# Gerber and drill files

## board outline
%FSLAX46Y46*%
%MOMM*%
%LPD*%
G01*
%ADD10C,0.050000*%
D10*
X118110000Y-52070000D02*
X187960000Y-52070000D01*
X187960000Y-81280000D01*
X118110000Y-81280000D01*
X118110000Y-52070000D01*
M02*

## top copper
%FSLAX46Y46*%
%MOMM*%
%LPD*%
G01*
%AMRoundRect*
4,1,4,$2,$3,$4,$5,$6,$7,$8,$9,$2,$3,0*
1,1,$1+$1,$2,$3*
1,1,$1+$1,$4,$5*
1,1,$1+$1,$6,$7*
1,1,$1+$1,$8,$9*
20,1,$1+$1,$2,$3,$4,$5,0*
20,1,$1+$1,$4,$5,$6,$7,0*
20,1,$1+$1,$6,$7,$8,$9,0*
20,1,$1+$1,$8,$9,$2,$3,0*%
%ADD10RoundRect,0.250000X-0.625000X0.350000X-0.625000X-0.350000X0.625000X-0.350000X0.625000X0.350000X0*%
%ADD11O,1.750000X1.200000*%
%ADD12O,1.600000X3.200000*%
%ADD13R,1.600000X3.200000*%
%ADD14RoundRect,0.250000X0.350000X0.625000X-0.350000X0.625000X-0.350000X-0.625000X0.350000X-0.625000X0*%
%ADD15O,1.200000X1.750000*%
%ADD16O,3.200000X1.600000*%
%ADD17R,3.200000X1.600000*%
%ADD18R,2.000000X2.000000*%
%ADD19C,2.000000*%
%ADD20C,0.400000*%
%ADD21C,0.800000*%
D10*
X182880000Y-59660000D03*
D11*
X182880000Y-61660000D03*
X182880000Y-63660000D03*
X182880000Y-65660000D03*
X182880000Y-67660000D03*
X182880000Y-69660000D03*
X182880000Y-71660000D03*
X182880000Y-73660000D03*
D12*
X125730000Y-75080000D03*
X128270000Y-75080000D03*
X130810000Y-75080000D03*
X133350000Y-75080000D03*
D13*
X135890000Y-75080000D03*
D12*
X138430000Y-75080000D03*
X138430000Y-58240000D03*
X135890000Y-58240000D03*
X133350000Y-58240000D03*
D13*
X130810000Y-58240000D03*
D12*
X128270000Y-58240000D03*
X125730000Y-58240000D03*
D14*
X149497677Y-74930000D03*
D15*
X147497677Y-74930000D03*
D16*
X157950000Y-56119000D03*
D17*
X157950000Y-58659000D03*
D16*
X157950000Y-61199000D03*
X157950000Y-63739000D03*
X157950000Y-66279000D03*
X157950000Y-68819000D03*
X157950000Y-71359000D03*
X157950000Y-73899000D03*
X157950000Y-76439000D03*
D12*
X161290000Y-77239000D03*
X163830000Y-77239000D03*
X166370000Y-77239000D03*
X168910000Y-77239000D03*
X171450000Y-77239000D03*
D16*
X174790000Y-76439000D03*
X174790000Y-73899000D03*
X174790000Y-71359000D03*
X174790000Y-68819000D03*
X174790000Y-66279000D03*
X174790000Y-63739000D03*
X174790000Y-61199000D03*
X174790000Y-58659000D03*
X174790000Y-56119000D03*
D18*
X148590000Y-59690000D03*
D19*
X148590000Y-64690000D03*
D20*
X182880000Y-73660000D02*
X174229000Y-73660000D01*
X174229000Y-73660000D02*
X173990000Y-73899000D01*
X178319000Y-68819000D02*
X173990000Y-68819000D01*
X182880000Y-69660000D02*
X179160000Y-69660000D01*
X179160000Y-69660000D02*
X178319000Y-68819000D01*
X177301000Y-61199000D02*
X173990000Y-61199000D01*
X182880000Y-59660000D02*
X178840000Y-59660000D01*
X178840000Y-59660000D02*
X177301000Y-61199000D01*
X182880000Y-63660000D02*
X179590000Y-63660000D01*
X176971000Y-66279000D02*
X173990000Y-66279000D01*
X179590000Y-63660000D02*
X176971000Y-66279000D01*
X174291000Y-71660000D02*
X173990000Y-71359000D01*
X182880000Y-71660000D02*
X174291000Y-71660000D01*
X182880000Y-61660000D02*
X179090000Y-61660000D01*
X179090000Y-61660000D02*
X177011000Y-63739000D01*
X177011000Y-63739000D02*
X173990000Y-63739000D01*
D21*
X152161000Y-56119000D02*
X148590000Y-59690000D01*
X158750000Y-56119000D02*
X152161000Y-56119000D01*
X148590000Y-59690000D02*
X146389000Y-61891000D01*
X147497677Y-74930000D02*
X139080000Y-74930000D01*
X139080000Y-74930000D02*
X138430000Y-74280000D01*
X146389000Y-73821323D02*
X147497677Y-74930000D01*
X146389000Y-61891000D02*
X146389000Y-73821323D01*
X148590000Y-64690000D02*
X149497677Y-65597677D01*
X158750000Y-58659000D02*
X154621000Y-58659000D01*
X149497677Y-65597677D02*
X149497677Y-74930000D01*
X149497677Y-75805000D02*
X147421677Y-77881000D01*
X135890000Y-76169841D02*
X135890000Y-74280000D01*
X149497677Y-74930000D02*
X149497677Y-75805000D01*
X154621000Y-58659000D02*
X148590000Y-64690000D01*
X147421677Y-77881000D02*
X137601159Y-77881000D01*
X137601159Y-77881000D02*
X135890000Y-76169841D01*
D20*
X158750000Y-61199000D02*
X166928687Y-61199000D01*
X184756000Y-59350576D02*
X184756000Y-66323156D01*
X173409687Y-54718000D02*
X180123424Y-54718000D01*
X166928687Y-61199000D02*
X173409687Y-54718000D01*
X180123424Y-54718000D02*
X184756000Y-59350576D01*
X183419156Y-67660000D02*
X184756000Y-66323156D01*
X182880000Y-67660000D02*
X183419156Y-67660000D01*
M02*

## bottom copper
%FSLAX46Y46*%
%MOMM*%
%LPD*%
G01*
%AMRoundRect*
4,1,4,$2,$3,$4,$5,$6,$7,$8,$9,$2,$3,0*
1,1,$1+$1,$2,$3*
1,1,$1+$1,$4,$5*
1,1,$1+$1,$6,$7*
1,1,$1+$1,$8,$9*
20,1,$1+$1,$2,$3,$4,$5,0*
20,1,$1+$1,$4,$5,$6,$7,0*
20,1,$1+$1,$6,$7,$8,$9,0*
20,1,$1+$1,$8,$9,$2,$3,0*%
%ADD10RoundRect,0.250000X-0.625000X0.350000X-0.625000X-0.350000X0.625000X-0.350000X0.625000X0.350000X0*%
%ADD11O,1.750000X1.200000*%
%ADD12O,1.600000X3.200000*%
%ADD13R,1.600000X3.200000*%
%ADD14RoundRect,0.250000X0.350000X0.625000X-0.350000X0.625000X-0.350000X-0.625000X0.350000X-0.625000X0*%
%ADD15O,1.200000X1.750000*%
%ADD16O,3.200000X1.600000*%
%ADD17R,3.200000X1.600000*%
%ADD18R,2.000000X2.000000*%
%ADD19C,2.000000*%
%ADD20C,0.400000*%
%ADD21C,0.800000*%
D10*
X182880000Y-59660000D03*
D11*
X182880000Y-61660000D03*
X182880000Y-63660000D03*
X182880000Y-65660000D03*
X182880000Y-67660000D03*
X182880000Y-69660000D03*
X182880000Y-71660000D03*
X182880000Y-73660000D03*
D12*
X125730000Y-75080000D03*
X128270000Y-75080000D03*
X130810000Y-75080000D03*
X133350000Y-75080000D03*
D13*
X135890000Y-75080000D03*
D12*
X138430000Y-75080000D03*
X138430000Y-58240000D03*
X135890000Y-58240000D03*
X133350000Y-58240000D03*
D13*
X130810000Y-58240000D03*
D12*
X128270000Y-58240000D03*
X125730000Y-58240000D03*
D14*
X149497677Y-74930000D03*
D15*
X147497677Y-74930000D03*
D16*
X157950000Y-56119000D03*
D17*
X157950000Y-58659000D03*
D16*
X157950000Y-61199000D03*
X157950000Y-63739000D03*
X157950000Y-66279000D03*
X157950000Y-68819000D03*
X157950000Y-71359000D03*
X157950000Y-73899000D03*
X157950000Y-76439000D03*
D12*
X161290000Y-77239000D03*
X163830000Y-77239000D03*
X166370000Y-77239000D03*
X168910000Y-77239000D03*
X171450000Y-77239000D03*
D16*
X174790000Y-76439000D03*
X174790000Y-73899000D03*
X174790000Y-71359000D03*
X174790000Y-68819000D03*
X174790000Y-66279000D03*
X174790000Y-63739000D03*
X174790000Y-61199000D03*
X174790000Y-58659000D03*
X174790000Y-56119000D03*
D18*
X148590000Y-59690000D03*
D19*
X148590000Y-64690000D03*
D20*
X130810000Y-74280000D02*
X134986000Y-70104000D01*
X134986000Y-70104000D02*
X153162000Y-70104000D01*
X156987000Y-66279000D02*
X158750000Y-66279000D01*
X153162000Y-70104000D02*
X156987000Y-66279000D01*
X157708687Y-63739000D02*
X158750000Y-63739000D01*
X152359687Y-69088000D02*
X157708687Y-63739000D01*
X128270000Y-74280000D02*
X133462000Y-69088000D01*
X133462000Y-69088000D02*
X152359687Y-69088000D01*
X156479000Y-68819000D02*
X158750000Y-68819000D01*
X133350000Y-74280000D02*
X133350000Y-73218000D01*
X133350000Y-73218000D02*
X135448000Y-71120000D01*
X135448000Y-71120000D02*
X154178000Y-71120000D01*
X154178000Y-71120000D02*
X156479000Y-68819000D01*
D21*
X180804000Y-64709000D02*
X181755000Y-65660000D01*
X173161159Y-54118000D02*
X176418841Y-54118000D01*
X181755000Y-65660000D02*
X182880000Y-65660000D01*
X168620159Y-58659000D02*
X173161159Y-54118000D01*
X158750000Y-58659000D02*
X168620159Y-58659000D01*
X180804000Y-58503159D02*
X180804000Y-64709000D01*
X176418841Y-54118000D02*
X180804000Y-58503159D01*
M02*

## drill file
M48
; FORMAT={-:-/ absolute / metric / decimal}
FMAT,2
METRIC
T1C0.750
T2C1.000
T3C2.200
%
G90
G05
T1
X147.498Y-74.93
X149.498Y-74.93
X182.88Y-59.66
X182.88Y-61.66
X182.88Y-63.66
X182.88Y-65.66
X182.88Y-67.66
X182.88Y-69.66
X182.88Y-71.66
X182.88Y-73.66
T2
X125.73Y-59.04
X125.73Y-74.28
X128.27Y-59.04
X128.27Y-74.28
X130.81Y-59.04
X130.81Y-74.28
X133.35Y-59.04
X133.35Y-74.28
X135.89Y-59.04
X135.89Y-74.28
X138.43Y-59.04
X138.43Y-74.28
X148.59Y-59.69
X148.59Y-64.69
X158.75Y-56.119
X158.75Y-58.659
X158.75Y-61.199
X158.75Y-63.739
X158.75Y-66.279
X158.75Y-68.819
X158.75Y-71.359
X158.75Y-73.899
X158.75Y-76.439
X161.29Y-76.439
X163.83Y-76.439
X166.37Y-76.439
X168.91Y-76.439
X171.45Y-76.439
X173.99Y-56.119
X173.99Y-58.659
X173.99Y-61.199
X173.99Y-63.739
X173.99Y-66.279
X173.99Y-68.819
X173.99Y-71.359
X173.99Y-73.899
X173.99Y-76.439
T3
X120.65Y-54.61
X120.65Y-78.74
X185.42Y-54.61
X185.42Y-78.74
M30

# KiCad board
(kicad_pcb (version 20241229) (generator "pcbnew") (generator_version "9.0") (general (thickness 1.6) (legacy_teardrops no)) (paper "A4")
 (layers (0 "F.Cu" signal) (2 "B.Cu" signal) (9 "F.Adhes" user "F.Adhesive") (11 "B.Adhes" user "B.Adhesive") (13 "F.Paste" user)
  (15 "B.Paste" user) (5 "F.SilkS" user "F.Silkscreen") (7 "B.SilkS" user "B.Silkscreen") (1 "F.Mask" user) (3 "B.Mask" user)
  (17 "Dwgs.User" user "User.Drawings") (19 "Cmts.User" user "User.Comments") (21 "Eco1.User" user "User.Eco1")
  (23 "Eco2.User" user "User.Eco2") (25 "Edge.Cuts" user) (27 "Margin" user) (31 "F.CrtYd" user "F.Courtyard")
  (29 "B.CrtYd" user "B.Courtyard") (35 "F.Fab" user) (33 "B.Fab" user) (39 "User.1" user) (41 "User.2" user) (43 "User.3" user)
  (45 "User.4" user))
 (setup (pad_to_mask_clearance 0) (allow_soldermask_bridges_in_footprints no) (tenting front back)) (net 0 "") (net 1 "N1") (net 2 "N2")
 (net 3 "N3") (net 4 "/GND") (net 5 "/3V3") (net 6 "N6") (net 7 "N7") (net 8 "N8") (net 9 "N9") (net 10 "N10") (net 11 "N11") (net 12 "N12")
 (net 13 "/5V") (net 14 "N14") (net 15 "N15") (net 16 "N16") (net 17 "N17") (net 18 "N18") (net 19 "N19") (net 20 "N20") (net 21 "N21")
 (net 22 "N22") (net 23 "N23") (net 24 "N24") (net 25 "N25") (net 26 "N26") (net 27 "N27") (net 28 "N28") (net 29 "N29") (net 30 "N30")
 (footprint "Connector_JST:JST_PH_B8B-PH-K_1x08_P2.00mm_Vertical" (layer "F.Cu") (at 182.88 59.66 -90)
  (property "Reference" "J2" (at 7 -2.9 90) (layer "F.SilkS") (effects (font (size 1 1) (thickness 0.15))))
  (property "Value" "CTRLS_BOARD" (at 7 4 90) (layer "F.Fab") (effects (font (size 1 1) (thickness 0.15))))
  (pad "1" thru_hole roundrect (at 0 0 270) (size 1.2 1.75) (drill 0.75) (layers "*.Cu" "*.Mask") (remove_unused_layers no)
   (roundrect_rratio 0.208333) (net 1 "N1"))
  (pad "2" thru_hole oval (at 2 0 270) (size 1.2 1.75) (drill 0.75) (layers "*.Cu" "*.Mask") (remove_unused_layers no) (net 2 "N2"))
  (pad "3" thru_hole oval (at 4 0 270) (size 1.2 1.75) (drill 0.75) (layers "*.Cu" "*.Mask") (remove_unused_layers no) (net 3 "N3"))
  (pad "4" thru_hole oval (at 6 0 270) (size 1.2 1.75) (drill 0.75) (layers "*.Cu" "*.Mask") (remove_unused_layers no) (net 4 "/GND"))
  (pad "5" thru_hole oval (at 8 0 270) (size 1.2 1.75) (drill 0.75) (layers "*.Cu" "*.Mask") (remove_unused_layers no) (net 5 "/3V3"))
  (pad "6" thru_hole oval (at 10 0 270) (size 1.2 1.75) (drill 0.75) (layers "*.Cu" "*.Mask") (remove_unused_layers no) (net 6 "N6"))
  (pad "7" thru_hole oval (at 12 0 270) (size 1.2 1.75) (drill 0.75) (layers "*.Cu" "*.Mask") (remove_unused_layers no) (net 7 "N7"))
  (pad "8" thru_hole oval (at 14 0 270) (size 1.2 1.75) (drill 0.75) (layers "*.Cu" "*.Mask") (remove_unused_layers no) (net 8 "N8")))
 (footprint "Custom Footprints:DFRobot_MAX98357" (layer "F.Cu") (at 140.97 66.66 90)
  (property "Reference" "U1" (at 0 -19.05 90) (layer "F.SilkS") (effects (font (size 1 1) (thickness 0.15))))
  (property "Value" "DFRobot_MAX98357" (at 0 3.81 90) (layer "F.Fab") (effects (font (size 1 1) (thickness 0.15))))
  (pad "1" thru_hole oval (at -7.62 -15.24 90) (size 3.2 1.6) (drill 1 (offset -0.8 0)) (layers "*.Cu" "*.Mask") (remove_unused_layers no)
   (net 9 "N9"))
  (pad "2" thru_hole oval (at -7.62 -12.7 90) (size 3.2 1.6) (drill 1 (offset -0.8 0)) (layers "*.Cu" "*.Mask") (remove_unused_layers no)
   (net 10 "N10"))
  (pad "3" thru_hole oval (at -7.62 -10.16 90) (size 3.2 1.6) (drill 1 (offset -0.8 0)) (layers "*.Cu" "*.Mask") (remove_unused_layers no)
   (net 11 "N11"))
  (pad "4" thru_hole oval (at -7.62 -7.62 90) (size 3.2 1.6) (drill 1 (offset -0.8 0)) (layers "*.Cu" "*.Mask") (remove_unused_layers no)
   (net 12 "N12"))
  (pad "5" thru_hole rect (at -7.62 -5.08 90) (size 3.2 1.6) (drill 1 (offset -0.8 0)) (layers "*.Cu" "*.Mask") (remove_unused_layers no)
   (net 4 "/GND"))
  (pad "6" thru_hole oval (at -7.62 -2.54 90) (size 3.2 1.6) (drill 1 (offset -0.8 0)) (layers "*.Cu" "*.Mask") (remove_unused_layers no)
   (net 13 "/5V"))
  (pad "7" thru_hole oval (at 7.62 -2.54 90) (size 3.2 1.6) (drill 1 (offset 0.8 0)) (layers "*.Cu" "*.Mask") (remove_unused_layers no)
   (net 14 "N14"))
  (pad "8" thru_hole oval (at 7.62 -5.08 90) (size 3.2 1.6) (drill 1 (offset 0.8 0)) (layers "*.Cu" "*.Mask") (remove_unused_layers no)
   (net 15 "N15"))
  (pad "9" thru_hole oval (at 7.62 -7.62 90) (size 3.2 1.6) (drill 1 (offset 0.8 0)) (layers "*.Cu" "*.Mask") (remove_unused_layers no)
   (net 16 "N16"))
  (pad "10" thru_hole rect (at 7.62 -10.16 90) (size 3.2 1.6) (drill 1 (offset 0.8 0)) (layers "*.Cu" "*.Mask") (remove_unused_layers no)
   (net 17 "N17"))
  (pad "11" thru_hole oval (at 7.62 -12.7 90) (size 3.2 1.6) (drill 1 (offset 0.8 0)) (layers "*.Cu" "*.Mask") (remove_unused_layers no)
   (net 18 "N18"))
  (pad "12" thru_hole oval (at 7.62 -15.24 90) (size 3.2 1.6) (drill 1 (offset 0.8 0)) (layers "*.Cu" "*.Mask") (remove_unused_layers no)
   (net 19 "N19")))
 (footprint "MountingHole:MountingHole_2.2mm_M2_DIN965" (layer "F.Cu") (at 185.42 54.61)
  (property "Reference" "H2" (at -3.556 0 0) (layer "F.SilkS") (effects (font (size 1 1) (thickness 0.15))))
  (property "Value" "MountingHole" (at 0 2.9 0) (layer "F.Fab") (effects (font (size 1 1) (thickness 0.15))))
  (pad "" np_thru_hole circle (at 0 0) (size 2.2 2.2) (drill 2.2) (layers "*.Cu" "*.Mask")))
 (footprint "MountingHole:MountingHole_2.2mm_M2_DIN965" (layer "F.Cu") (at 185.42 78.74)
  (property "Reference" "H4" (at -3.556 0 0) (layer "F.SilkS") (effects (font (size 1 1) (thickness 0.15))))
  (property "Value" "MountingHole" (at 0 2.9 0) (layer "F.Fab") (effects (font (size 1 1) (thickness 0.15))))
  (pad "" np_thru_hole circle (at 0 0) (size 2.2 2.2) (drill 2.2) (layers "*.Cu" "*.Mask")))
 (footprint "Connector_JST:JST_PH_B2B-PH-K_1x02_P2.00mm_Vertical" (layer "F.Cu") (at 149.497677 74.93 180)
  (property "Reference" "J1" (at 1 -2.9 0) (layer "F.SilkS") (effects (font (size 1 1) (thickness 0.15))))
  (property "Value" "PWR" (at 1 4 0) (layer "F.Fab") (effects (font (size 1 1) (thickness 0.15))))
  (pad "1" thru_hole roundrect (at 0 0 180) (size 1.2 1.75) (drill 0.75) (layers "*.Cu" "*.Mask") (remove_unused_layers no)
   (roundrect_rratio 0.208333) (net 4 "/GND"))
  (pad "2" thru_hole oval (at 2 0 180) (size 1.2 1.75) (drill 0.75) (layers "*.Cu" "*.Mask") (remove_unused_layers no) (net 13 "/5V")))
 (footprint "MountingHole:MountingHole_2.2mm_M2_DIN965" (layer "F.Cu") (at 120.65 54.61)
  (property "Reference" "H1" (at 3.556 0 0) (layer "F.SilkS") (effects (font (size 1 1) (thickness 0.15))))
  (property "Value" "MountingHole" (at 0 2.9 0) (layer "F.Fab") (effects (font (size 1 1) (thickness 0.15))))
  (pad "" np_thru_hole circle (at 0 0) (size 2.2 2.2) (drill 2.2) (layers "*.Cu" "*.Mask")))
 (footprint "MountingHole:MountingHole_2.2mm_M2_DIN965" (layer "F.Cu") (at 120.65 78.74)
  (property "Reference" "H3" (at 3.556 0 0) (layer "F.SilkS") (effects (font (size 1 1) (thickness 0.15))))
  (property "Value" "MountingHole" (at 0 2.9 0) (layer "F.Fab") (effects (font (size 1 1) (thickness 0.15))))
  (pad "" np_thru_hole circle (at 0 0) (size 2.2 2.2) (drill 2.2) (layers "*.Cu" "*.Mask")))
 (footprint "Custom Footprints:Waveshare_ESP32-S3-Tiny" (layer "F.Cu") (at 158.75 56.119)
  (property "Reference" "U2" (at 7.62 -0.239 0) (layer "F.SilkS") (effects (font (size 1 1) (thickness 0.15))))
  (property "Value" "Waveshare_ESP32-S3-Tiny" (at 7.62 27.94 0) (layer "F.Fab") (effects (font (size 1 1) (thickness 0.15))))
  (pad "1" thru_hole oval (at 0 0) (size 3.2 1.6) (drill 1 (offset -0.8 0)) (layers "*.Cu" "*.Mask") (remove_unused_layers no)
   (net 13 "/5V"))
  (pad "2" thru_hole rect (at 0 2.54) (size 3.2 1.6) (drill 1 (offset -0.8 0)) (layers "*.Cu" "*.Mask") (remove_unused_layers no)
   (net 4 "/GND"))
  (pad "3" thru_hole oval (at 0 5.08) (size 3.2 1.6) (drill 1 (offset -0.8 0)) (layers "*.Cu" "*.Mask") (remove_unused_layers no)
   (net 5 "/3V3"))
  (pad "4" thru_hole oval (at 0 7.62) (size 3.2 1.6) (drill 1 (offset -0.8 0)) (layers "*.Cu" "*.Mask") (remove_unused_layers no)
   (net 10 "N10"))
  (pad "5" thru_hole oval (at 0 10.16) (size 3.2 1.6) (drill 1 (offset -0.8 0)) (layers "*.Cu" "*.Mask") (remove_unused_layers no)
   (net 11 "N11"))
  (pad "6" thru_hole oval (at 0 12.7) (size 3.2 1.6) (drill 1 (offset -0.8 0)) (layers "*.Cu" "*.Mask") (remove_unused_layers no)
   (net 12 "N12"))
  (pad "7" thru_hole oval (at 0 15.24) (size 3.2 1.6) (drill 1 (offset -0.8 0)) (layers "*.Cu" "*.Mask") (remove_unused_layers no)
   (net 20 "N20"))
  (pad "8" thru_hole oval (at 0 17.78) (size 3.2 1.6) (drill 1 (offset -0.8 0)) (layers "*.Cu" "*.Mask") (remove_unused_layers no)
   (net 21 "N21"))
  (pad "9" thru_hole oval (at 0 20.32) (size 3.2 1.6) (drill 1 (offset -0.8 0)) (layers "*.Cu" "*.Mask") (remove_unused_layers no)
   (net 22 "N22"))
  (pad "10" thru_hole oval (at 2.54 20.32) (size 1.6 3.2) (drill 1 (offset 0 0.8)) (layers "*.Cu" "*.Mask") (remove_unused_layers no)
   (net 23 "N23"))
  (pad "11" thru_hole oval (at 5.08 20.32) (size 1.6 3.2) (drill 1 (offset 0 0.8)) (layers "*.Cu" "*.Mask") (remove_unused_layers no)
   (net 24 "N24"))
  (pad "12" thru_hole oval (at 7.62 20.32) (size 1.6 3.2) (drill 1 (offset 0 0.8)) (layers "*.Cu" "*.Mask") (remove_unused_layers no)
   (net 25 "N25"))
  (pad "13" thru_hole oval (at 10.16 20.32) (size 1.6 3.2) (drill 1 (offset 0 0.8)) (layers "*.Cu" "*.Mask") (remove_unused_layers no)
   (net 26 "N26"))
  (pad "14" thru_hole oval (at 12.7 20.32) (size 1.6 3.2) (drill 1 (offset 0 0.8)) (layers "*.Cu" "*.Mask") (remove_unused_layers no)
   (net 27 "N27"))
  (pad "15" thru_hole oval (at 15.24 20.32) (size 3.2 1.6) (drill 1 (offset 0.8 0)) (layers "*.Cu" "*.Mask") (remove_unused_layers no)
   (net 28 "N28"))
  (pad "16" thru_hole oval (at 15.24 17.78) (size 3.2 1.6) (drill 1 (offset 0.8 0)) (layers "*.Cu" "*.Mask") (remove_unused_layers no)
   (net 8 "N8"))
  (pad "17" thru_hole oval (at 15.24 15.24) (size 3.2 1.6) (drill 1 (offset 0.8 0)) (layers "*.Cu" "*.Mask") (remove_unused_layers no)
   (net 7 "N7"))
  (pad "18" thru_hole oval (at 15.24 12.7) (size 3.2 1.6) (drill 1 (offset 0.8 0)) (layers "*.Cu" "*.Mask") (remove_unused_layers no)
   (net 6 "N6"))
  (pad "19" thru_hole oval (at 15.24 10.16) (size 3.2 1.6) (drill 1 (offset 0.8 0)) (layers "*.Cu" "*.Mask") (remove_unused_layers no)
   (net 3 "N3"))
  (pad "20" thru_hole oval (at 15.24 7.62) (size 3.2 1.6) (drill 1 (offset 0.8 0)) (layers "*.Cu" "*.Mask") (remove_unused_layers no)
   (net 2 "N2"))
  (pad "21" thru_hole oval (at 15.24 5.08) (size 3.2 1.6) (drill 1 (offset 0.8 0)) (layers "*.Cu" "*.Mask") (remove_unused_layers no)
   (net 1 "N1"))
  (pad "22" thru_hole oval (at 15.24 2.54) (size 3.2 1.6) (drill 1 (offset 0.8 0)) (layers "*.Cu" "*.Mask") (remove_unused_layers no)
   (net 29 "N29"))
  (pad "23" thru_hole oval (at 15.24 0) (size 3.2 1.6) (drill 1 (offset 0.8 0)) (layers "*.Cu" "*.Mask") (remove_unused_layers no)
   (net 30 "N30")))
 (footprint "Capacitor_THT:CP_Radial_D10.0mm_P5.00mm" (layer "F.Cu") (at 148.59 59.69 -90)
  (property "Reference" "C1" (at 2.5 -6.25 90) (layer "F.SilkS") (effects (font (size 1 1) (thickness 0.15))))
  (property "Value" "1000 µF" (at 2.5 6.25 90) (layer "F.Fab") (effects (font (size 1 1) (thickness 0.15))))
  (pad "1" thru_hole rect (at 0 0 270) (size 2 2) (drill 1) (layers "*.Cu" "*.Mask") (remove_unused_layers no) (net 13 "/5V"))
  (pad "2" thru_hole circle (at 5 0 270) (size 2 2) (drill 1) (layers "*.Cu" "*.Mask") (remove_unused_layers no) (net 4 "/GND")))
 (gr_rect (start 118.11 52.07) (end 187.96 81.28) (stroke (width 0.05) (type default)) (fill no) (layer "Edge.Cuts"))
 (segment (start 182.88 73.66) (end 174.229 73.66) (width 0.4) (layer "F.Cu") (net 8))
 (segment (start 174.229 73.66) (end 173.99 73.899) (width 0.4) (layer "F.Cu") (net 8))
 (segment (start 178.319 68.819) (end 173.99 68.819) (width 0.4) (layer "F.Cu") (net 6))
 (segment (start 182.88 69.66) (end 179.16 69.66) (width 0.4) (layer "F.Cu") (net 6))
 (segment (start 179.16 69.66) (end 178.319 68.819) (width 0.4) (layer "F.Cu") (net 6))
 (segment (start 177.301 61.199) (end 173.99 61.199) (width 0.4) (layer "F.Cu") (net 1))
 (segment (start 182.88 59.66) (end 178.84 59.66) (width 0.4) (layer "F.Cu") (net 1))
 (segment (start 178.84 59.66) (end 177.301 61.199) (width 0.4) (layer "F.Cu") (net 1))
 (segment (start 182.88 63.66) (end 179.59 63.66) (width 0.4) (layer "F.Cu") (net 3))
 (segment (start 176.971 66.279) (end 173.99 66.279) (width 0.4) (layer "F.Cu") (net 3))
 (segment (start 179.59 63.66) (end 176.971 66.279) (width 0.4) (layer "F.Cu") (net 3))
 (segment (start 174.291 71.66) (end 173.99 71.359) (width 0.4) (layer "F.Cu") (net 7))
 (segment (start 182.88 71.66) (end 174.291 71.66) (width 0.4) (layer "F.Cu") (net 7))
 (segment (start 182.88 61.66) (end 179.09 61.66) (width 0.4) (layer "F.Cu") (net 2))
 (segment (start 179.09 61.66) (end 177.011 63.739) (width 0.4) (layer "F.Cu") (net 2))
 (segment (start 177.011 63.739) (end 173.99 63.739) (width 0.4) (layer "F.Cu") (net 2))
 (segment (start 130.81 74.28) (end 134.986 70.104) (width 0.4) (layer "B.Cu") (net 11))
 (segment (start 134.986 70.104) (end 153.162 70.104) (width 0.4) (layer "B.Cu") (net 11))
 (segment (start 156.987 66.279) (end 158.75 66.279) (width 0.4) (layer "B.Cu") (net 11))
 (segment (start 153.162 70.104) (end 156.987 66.279) (width 0.4) (layer "B.Cu") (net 11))
 (segment (start 157.708687 63.739) (end 158.75 63.739) (width 0.4) (layer "B.Cu") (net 10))
 (segment (start 152.359687 69.088) (end 157.708687 63.739) (width 0.4) (layer "B.Cu") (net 10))
 (segment (start 128.27 74.28) (end 133.462 69.088) (width 0.4) (layer "B.Cu") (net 10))
 (segment (start 133.462 69.088) (end 152.359687 69.088) (width 0.4) (layer "B.Cu") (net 10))
 (segment (start 156.479 68.819) (end 158.75 68.819) (width 0.4) (layer "B.Cu") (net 12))
 (segment (start 133.35 74.28) (end 133.35 73.218) (width 0.4) (layer "B.Cu") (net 12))
 (segment (start 133.35 73.218) (end 135.448 71.12) (width 0.4) (layer "B.Cu") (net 12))
 (segment (start 135.448 71.12) (end 154.178 71.12) (width 0.4) (layer "B.Cu") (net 12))
 (segment (start 154.178 71.12) (end 156.479 68.819) (width 0.4) (layer "B.Cu") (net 12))
 (segment (start 152.161 56.119) (end 148.59 59.69) (width 0.8) (layer "F.Cu") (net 13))
 (segment (start 158.75 56.119) (end 152.161 56.119) (width 0.8) (layer "F.Cu") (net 13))
 (segment (start 148.59 59.69) (end 146.389 61.891) (width 0.8) (layer "F.Cu") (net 13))
 (segment (start 147.497677 74.93) (end 139.08 74.93) (width 0.8) (layer "F.Cu") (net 13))
 (segment (start 139.08 74.93) (end 138.43 74.28) (width 0.8) (layer "F.Cu") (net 13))
 (segment (start 146.389 73.821323) (end 147.497677 74.93) (width 0.8) (layer "F.Cu") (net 13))
 (segment (start 146.389 61.891) (end 146.389 73.821323) (width 0.8) (layer "F.Cu") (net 13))
 (segment (start 148.59 64.69) (end 149.497677 65.597677) (width 0.8) (layer "F.Cu") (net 4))
 (segment (start 158.75 58.659) (end 154.621 58.659) (width 0.8) (layer "F.Cu") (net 4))
 (segment (start 149.497677 65.597677) (end 149.497677 74.93) (width 0.8) (layer "F.Cu") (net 4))
 (segment (start 149.497677 75.805) (end 147.421677 77.881) (width 0.8) (layer "F.Cu") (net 4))
 (segment (start 135.89 76.169841) (end 135.89 74.28) (width 0.8) (layer "F.Cu") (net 4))
 (segment (start 149.497677 74.93) (end 149.497677 75.805) (width 0.8) (layer "F.Cu") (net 4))
 (segment (start 154.621 58.659) (end 148.59 64.69) (width 0.8) (layer "F.Cu") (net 4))
 (segment (start 147.421677 77.881) (end 137.601159 77.881) (width 0.8) (layer "F.Cu") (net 4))
 (segment (start 137.601159 77.881) (end 135.89 76.169841) (width 0.8) (layer "F.Cu") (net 4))
 (segment (start 180.804 64.709) (end 181.755 65.66) (width 0.8) (layer "B.Cu") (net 4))
 (segment (start 173.161159 54.118) (end 176.418841 54.118) (width 0.8) (layer "B.Cu") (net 4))
 (segment (start 181.755 65.66) (end 182.88 65.66) (width 0.8) (layer "B.Cu") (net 4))
 (segment (start 168.620159 58.659) (end 173.161159 54.118) (width 0.8) (layer "B.Cu") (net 4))
 (segment (start 158.75 58.659) (end 168.620159 58.659) (width 0.8) (layer "B.Cu") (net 4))
 (segment (start 180.804 58.503159) (end 180.804 64.709) (width 0.8) (layer "B.Cu") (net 4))
 (segment (start 176.418841 54.118) (end 180.804 58.503159) (width 0.8) (layer "B.Cu") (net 4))
 (segment (start 158.75 61.199) (end 166.928687 61.199) (width 0.4) (layer "F.Cu") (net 5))
 (segment (start 184.756 59.350576) (end 184.756 66.323156) (width 0.4) (layer "F.Cu") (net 5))
 (segment (start 173.409687 54.718) (end 180.123424 54.718) (width 0.4) (layer "F.Cu") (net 5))
 (segment (start 166.928687 61.199) (end 173.409687 54.718) (width 0.4) (layer "F.Cu") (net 5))
 (segment (start 180.123424 54.718) (end 184.756 59.350576) (width 0.4) (layer "F.Cu") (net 5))
 (segment (start 183.419156 67.66) (end 184.756 66.323156) (width 0.4) (layer "F.Cu") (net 5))
 (segment (start 182.88 67.66) (end 183.419156 67.66) (width 0.4) (layer "F.Cu") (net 5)))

